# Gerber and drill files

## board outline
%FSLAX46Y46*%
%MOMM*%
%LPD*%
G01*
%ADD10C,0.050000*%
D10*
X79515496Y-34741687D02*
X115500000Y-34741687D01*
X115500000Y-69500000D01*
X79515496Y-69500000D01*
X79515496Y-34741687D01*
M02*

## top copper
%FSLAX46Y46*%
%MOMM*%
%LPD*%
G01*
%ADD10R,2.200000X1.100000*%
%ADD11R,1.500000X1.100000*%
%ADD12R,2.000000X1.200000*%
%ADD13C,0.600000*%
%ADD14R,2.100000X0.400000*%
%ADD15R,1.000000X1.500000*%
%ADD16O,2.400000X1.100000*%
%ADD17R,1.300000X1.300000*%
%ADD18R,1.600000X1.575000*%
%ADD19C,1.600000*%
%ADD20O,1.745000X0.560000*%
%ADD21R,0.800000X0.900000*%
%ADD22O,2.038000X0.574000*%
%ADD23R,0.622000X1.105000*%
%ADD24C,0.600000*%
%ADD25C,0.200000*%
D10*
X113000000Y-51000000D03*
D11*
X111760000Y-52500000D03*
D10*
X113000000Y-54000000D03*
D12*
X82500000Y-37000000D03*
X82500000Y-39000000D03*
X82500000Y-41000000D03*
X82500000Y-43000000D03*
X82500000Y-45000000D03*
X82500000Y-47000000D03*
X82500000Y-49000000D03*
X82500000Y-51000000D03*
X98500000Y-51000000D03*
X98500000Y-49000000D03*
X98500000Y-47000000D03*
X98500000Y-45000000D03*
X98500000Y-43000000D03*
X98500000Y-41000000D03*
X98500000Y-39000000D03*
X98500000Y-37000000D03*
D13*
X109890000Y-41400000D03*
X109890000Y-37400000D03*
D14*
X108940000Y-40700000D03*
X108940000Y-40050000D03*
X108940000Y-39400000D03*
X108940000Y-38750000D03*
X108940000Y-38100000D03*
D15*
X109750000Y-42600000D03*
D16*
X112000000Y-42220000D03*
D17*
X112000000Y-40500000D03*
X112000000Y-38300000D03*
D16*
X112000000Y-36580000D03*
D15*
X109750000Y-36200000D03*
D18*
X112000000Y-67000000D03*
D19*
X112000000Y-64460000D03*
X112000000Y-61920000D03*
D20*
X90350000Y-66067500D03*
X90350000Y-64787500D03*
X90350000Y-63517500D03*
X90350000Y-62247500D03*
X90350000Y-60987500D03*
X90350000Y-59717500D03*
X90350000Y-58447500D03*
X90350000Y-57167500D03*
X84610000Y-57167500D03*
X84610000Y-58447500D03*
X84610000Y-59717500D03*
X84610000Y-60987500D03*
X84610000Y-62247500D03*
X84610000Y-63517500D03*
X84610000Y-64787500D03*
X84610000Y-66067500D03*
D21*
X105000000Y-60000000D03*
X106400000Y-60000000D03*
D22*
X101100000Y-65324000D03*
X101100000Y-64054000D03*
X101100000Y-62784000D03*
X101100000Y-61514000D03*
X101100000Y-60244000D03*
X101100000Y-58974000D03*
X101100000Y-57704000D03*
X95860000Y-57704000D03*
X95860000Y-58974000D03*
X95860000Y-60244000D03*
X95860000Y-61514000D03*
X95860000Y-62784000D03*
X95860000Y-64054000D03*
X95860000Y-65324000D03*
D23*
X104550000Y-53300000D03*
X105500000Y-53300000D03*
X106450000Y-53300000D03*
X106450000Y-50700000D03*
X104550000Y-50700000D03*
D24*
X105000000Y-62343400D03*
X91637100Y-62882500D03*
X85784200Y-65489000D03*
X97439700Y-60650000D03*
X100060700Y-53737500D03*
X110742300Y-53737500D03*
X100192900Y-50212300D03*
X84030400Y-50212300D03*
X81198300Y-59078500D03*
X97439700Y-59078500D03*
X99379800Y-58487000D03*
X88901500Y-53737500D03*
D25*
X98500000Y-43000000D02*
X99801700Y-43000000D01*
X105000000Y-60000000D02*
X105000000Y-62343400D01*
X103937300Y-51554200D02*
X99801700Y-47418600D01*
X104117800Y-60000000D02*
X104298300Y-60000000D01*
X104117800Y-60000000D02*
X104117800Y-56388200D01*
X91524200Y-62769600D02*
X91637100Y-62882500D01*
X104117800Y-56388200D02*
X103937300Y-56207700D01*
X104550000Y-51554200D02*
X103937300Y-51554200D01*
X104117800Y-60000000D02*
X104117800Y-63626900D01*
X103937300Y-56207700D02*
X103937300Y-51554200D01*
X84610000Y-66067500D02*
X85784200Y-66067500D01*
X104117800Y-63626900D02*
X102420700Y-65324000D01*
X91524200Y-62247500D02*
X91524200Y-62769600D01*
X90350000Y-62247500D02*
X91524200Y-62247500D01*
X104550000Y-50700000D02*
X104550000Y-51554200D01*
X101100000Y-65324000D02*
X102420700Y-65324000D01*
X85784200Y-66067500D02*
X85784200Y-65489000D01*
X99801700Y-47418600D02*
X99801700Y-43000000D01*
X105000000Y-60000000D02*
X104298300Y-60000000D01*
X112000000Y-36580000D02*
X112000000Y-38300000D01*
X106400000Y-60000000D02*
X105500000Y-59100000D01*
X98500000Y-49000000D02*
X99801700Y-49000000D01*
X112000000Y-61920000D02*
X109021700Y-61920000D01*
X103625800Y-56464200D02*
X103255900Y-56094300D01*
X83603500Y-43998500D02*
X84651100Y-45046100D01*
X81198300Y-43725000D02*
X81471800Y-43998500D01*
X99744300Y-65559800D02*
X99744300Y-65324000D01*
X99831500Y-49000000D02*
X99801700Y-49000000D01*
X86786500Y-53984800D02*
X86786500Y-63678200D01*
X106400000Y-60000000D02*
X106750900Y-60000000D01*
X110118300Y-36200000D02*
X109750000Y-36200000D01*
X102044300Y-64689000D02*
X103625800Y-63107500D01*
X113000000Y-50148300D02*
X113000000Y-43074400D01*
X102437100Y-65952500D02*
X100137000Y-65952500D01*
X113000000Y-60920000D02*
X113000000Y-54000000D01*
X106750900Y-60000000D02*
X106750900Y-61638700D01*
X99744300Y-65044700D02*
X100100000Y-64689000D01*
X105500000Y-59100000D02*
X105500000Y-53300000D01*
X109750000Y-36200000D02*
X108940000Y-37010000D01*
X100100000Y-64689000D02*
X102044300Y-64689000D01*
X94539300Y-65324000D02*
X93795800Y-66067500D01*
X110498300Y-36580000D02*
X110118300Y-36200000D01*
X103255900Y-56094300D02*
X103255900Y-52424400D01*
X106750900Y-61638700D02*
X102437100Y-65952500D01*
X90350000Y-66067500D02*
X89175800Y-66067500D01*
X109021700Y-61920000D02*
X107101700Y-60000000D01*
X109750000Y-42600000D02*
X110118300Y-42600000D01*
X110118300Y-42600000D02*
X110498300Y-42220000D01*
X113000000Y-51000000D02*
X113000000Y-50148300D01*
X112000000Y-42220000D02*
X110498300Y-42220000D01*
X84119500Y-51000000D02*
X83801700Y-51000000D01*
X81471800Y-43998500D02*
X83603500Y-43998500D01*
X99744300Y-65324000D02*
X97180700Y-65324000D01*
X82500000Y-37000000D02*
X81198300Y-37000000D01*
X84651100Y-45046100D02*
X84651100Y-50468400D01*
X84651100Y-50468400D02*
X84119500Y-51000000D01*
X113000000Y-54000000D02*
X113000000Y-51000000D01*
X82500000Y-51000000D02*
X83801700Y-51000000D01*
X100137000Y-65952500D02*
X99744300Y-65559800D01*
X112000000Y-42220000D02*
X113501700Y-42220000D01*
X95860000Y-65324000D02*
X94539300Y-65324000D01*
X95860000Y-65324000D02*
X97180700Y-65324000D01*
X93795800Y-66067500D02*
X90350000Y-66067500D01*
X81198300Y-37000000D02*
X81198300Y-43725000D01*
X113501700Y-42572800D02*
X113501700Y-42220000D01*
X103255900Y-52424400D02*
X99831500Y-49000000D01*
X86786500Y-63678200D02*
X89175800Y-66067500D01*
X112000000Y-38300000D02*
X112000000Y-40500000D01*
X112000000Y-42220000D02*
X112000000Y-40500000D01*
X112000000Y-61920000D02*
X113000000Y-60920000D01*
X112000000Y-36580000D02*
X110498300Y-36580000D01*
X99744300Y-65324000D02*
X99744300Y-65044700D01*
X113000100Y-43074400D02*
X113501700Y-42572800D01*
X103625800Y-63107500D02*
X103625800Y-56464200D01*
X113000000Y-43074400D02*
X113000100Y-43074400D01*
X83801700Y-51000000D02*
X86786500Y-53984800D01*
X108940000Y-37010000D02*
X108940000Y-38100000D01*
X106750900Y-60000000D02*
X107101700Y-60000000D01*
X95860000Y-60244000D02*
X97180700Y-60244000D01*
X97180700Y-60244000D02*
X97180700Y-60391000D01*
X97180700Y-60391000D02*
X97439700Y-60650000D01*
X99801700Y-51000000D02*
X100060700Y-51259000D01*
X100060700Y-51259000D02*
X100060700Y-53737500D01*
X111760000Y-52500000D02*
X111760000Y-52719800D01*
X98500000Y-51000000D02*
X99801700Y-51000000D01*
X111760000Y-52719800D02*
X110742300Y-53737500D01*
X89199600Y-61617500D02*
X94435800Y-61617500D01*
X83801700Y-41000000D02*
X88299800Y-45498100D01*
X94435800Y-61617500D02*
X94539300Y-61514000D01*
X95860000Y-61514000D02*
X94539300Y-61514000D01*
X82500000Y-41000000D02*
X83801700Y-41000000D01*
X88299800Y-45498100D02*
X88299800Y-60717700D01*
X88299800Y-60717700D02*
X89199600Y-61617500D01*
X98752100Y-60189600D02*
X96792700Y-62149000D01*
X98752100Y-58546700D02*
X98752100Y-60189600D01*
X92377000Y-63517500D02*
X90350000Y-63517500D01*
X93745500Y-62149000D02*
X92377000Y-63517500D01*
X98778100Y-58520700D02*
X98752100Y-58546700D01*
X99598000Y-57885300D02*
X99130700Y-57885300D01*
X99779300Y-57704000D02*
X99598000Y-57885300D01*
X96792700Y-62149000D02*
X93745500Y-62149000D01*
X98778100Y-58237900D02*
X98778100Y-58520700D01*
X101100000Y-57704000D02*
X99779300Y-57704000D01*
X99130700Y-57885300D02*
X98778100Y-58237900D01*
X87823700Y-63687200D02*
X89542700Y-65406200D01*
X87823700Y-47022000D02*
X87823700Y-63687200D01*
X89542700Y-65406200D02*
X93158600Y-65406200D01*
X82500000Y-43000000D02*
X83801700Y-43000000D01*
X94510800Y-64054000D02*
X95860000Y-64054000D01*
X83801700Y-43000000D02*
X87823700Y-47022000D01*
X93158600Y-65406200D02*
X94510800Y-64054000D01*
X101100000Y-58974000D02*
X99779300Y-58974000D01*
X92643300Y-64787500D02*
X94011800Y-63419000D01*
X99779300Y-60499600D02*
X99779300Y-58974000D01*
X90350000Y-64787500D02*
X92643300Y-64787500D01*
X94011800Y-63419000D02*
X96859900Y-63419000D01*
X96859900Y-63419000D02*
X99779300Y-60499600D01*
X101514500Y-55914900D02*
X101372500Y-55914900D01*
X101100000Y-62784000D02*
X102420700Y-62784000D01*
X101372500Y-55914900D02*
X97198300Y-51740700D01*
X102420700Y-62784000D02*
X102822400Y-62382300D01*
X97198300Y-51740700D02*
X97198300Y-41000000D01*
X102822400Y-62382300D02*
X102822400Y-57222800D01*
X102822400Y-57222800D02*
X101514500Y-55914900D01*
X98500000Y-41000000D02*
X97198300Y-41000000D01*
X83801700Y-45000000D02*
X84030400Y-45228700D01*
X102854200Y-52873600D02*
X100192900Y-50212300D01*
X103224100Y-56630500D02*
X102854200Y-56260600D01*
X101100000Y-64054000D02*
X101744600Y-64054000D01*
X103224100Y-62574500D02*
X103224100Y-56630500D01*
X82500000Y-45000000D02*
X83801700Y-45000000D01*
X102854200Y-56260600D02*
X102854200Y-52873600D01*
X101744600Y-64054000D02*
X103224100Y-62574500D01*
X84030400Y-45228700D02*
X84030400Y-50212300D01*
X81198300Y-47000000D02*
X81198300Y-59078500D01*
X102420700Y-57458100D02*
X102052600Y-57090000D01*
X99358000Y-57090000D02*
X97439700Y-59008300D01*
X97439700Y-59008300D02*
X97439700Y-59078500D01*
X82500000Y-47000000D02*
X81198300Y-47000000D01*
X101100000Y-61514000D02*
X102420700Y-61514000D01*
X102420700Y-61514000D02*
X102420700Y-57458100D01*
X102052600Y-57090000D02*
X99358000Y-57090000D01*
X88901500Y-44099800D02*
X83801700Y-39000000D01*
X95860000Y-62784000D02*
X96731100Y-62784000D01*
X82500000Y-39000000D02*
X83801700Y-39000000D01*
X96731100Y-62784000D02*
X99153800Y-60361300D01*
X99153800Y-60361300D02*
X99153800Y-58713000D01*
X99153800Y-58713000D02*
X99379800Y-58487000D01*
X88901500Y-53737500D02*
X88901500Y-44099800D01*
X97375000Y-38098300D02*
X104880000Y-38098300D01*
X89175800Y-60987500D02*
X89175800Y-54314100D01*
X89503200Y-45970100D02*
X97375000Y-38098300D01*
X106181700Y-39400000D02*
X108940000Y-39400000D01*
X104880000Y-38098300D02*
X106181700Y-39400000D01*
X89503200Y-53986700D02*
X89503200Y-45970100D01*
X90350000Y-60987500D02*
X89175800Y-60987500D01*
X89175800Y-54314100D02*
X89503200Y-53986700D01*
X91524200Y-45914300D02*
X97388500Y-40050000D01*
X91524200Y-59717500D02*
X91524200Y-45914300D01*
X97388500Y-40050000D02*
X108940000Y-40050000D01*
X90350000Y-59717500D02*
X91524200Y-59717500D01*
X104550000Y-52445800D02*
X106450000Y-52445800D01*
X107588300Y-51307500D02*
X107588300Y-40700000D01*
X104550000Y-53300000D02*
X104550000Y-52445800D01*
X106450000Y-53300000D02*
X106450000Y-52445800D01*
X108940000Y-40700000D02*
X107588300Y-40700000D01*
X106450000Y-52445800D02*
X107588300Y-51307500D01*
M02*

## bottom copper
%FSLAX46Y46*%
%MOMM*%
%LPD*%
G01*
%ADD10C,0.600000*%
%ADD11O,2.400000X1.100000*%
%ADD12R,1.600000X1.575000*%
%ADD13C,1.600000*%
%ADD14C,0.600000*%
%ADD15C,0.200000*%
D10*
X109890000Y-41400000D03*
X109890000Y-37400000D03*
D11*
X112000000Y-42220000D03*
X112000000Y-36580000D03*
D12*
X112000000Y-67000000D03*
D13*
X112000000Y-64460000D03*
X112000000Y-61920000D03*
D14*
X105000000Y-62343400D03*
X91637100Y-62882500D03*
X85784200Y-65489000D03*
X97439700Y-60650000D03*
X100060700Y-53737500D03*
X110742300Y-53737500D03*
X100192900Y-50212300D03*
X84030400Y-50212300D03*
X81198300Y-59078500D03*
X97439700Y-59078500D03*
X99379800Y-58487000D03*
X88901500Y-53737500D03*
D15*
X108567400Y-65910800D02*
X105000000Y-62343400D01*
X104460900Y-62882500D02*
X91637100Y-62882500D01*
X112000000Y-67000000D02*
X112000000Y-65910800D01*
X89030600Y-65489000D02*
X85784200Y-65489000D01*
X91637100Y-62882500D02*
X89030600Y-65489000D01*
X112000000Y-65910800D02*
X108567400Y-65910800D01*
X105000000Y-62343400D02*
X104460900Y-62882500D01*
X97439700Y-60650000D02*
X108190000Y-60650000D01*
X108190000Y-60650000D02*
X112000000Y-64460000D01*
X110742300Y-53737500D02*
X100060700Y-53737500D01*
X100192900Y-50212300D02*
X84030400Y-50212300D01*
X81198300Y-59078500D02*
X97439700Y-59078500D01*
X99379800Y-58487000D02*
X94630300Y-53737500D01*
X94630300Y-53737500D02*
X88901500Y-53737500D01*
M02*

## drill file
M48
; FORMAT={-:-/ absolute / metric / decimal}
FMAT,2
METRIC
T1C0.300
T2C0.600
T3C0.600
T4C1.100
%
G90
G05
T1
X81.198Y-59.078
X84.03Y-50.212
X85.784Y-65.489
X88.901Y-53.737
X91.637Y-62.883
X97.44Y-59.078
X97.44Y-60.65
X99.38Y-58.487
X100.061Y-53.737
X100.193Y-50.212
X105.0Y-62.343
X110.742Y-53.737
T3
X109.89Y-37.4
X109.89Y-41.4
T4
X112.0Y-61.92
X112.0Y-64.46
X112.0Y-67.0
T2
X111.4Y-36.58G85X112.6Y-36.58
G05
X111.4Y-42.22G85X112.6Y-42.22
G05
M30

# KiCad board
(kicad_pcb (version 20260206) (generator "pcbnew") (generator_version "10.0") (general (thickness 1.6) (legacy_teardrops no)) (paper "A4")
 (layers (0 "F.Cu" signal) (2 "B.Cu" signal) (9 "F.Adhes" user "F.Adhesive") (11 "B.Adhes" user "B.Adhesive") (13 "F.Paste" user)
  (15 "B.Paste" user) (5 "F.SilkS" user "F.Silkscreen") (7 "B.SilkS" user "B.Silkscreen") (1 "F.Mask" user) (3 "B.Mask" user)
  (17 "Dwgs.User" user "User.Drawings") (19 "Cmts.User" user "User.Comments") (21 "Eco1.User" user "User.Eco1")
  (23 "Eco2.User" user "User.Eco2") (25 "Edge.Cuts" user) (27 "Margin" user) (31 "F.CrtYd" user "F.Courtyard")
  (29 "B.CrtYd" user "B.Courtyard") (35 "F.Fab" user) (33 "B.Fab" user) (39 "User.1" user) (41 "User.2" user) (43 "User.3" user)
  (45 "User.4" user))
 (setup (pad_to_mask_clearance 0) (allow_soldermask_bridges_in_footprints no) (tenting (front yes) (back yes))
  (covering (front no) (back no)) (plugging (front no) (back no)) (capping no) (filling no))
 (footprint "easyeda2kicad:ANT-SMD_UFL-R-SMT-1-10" (layer "F.Cu") (at 112.38 52.5)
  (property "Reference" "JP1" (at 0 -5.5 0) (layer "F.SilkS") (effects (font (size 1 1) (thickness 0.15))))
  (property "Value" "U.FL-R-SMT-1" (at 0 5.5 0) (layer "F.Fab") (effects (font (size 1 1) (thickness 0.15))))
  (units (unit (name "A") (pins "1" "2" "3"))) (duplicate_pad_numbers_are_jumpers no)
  (pad "1" smd rect (at 0.62 -1.5 270) (size 1.1 2.2) (layers "F.Cu" "F.Mask" "F.Paste") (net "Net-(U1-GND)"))
  (pad "2" smd rect (at -0.62 0) (size 1.5 1.1) (layers "F.Cu" "F.Mask" "F.Paste") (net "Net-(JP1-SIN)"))
  (pad "3" smd rect (at 0.62 1.5 270) (size 1.1 2.2) (layers "F.Cu" "F.Mask" "F.Paste") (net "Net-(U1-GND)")))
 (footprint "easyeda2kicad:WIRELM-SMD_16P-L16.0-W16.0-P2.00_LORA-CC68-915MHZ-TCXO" (layer "F.Cu") (at 90.5 44)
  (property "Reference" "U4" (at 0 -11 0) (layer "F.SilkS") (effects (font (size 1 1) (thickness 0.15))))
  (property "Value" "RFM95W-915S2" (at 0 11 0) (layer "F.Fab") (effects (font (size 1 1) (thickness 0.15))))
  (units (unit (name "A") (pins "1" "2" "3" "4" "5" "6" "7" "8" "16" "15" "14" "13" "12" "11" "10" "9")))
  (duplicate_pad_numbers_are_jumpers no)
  (pad "1" smd rect (at -8 -7 90) (size 1.2 2) (layers "F.Cu" "F.Mask" "F.Paste") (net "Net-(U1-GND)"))
  (pad "2" smd rect (at -8 -5 90) (size 1.2 2) (layers "F.Cu" "F.Mask" "F.Paste") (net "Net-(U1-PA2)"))
  (pad "3" smd rect (at -8 -3 90) (size 1.2 2) (layers "F.Cu" "F.Mask" "F.Paste") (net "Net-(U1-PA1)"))
  (pad "4" smd rect (at -8 -1 90) (size 1.2 2) (layers "F.Cu" "F.Mask" "F.Paste") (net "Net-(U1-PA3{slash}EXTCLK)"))
  (pad "5" smd rect (at -8 1 90) (size 1.2 2) (layers "F.Cu" "F.Mask" "F.Paste") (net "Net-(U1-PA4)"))
  (pad "6" smd rect (at -8 3 90) (size 1.2 2) (layers "F.Cu" "F.Mask" "F.Paste") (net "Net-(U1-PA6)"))
  (pad "7" smd rect (at -8 5 90) (size 1.2 2) (layers "F.Cu" "F.Mask" "F.Paste") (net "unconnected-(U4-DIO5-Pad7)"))
  (pad "8" smd rect (at -8 7 90) (size 1.2 2) (layers "F.Cu" "F.Mask" "F.Paste") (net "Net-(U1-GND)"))
  (pad "9" smd rect (at 8 7 90) (size 1.2 2) (layers "F.Cu" "F.Mask" "F.Paste") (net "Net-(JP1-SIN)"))
  (pad "10" smd rect (at 8 5 90) (size 1.2 2) (layers "F.Cu" "F.Mask" "F.Paste") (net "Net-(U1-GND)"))
  (pad "11" smd rect (at 8 3 90) (size 1.2 2) (layers "F.Cu" "F.Mask" "F.Paste") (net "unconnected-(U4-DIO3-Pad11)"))
  (pad "12" smd rect (at 8 1 90) (size 1.2 2) (layers "F.Cu" "F.Mask" "F.Paste") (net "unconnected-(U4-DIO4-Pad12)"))
  (pad "13" smd rect (at 8 -1 90) (size 1.2 2) (layers "F.Cu" "F.Mask" "F.Paste") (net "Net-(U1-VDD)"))
  (pad "14" smd rect (at 8 -3 90) (size 1.2 2) (layers "F.Cu" "F.Mask" "F.Paste") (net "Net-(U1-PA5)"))
  (pad "15" smd rect (at 8 -5 90) (size 1.2 2) (layers "F.Cu" "F.Mask" "F.Paste") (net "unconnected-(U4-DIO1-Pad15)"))
  (pad "16" smd rect (at 8 -7 90) (size 1.2 2) (layers "F.Cu" "F.Mask" "F.Paste") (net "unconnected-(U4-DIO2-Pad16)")))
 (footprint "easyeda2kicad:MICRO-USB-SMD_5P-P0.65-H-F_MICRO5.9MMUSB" (layer "F.Cu") (at 110.47 39.4 90)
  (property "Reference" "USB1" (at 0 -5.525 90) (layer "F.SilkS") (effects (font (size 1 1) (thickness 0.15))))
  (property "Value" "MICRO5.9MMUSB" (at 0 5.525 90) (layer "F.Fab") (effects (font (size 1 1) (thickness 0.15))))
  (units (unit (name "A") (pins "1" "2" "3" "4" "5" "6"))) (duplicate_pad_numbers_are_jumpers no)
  (pad "" thru_hole circle (at -2 -0.58 90) (size 0.6 0.6) (drill 0.6) (layers "*.Cu" "*.Mask") (remove_unused_layers no))
  (pad "" thru_hole circle (at 2 -0.58 90) (size 0.6 0.6) (drill 0.6) (layers "*.Cu" "*.Mask") (remove_unused_layers no))
  (pad "1" smd rect (at -1.3 -1.53 90) (size 0.4 2.1) (layers "F.Cu" "F.Mask" "F.Paste") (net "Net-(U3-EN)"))
  (pad "2" smd rect (at -0.65 -1.53 90) (size 0.4 2.1) (layers "F.Cu" "F.Mask" "F.Paste") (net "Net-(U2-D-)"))
  (pad "3" smd rect (at 0 -1.53 90) (size 0.4 2.1) (layers "F.Cu" "F.Mask" "F.Paste") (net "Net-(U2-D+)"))
  (pad "4" smd rect (at 0.65 -1.53 90) (size 0.4 2.1) (layers "F.Cu" "F.Mask" "F.Paste") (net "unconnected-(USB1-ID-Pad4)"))
  (pad "5" smd rect (at 1.3 -1.53 90) (size 0.4 2.1) (layers "F.Cu" "F.Mask" "F.Paste") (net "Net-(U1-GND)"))
  (pad "6" smd rect (at -3.2 -0.72 90) (size 1.5 1) (layers "F.Cu" "F.Mask" "F.Paste") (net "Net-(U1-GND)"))
  (pad "6" thru_hole oval (at -2.82 1.53 90) (size 1.1 2.4) (drill oval 0.599998 1.799996) (layers "*.Cu" "*.Mask")
   (remove_unused_layers no) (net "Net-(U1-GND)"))
  (pad "6" smd rect (at -1.1 1.53 90) (size 1.3 1.3) (layers "F.Cu" "F.Mask" "F.Paste") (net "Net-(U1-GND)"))
  (pad "6" smd rect (at 1.1 1.53 90) (size 1.3 1.3) (layers "F.Cu" "F.Mask" "F.Paste") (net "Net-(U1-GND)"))
  (pad "6" thru_hole oval (at 2.82 1.53 90) (size 1.1 2.4) (drill oval 0.599998 1.799996) (layers "*.Cu" "*.Mask") (remove_unused_layers no)
   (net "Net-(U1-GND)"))
  (pad "6" smd rect (at 3.2 -0.72 90) (size 1.5 1) (layers "F.Cu" "F.Mask" "F.Paste") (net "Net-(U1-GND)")))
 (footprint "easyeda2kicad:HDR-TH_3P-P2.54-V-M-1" (layer "F.Cu") (at 112 64.46 90)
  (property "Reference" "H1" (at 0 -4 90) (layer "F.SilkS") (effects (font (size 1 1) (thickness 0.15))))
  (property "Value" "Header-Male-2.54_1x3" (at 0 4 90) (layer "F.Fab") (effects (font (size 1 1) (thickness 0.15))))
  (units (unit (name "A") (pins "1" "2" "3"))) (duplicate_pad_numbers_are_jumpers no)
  (pad "1" thru_hole rect (at -2.54 0 90) (size 1.575 1.6) (drill 1.100024) (layers "*.Cu" "*.Mask") (remove_unused_layers no)
   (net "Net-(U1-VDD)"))
  (pad "2" thru_hole circle (at 0 0 90) (size 1.6 1.6) (drill 1.100024) (layers "*.Cu" "*.Mask") (remove_unused_layers no)
   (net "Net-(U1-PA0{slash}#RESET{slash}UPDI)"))
  (pad "3" thru_hole circle (at 2.54 0 90) (size 1.6 1.6) (drill 1.100024) (layers "*.Cu" "*.Mask") (remove_unused_layers no)
   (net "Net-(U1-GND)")))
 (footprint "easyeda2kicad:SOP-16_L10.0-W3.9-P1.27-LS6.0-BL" (layer "F.Cu") (at 87.48 61.6175 90)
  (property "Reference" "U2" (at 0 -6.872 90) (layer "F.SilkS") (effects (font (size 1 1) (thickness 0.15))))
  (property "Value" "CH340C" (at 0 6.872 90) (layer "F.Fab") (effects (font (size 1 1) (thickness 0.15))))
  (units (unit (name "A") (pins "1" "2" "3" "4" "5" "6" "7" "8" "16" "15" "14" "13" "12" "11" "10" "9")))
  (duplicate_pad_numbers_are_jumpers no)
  (pad "1" smd oval (at -4.45 2.87 90) (size 0.56 1.745) (layers "F.Cu" "F.Mask" "F.Paste") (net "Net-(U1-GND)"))
  (pad "2" smd oval (at -3.17 2.87 90) (size 0.56 1.745) (layers "F.Cu" "F.Mask" "F.Paste") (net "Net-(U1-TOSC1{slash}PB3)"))
  (pad "3" smd oval (at -1.9 2.87 90) (size 0.56 1.745) (layers "F.Cu" "F.Mask" "F.Paste") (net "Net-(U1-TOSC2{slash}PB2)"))
  (pad "4" smd oval (at -0.63 2.87 90) (size 0.56 1.745) (layers "F.Cu" "F.Mask" "F.Paste") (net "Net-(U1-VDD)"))
  (pad "5" smd oval (at 0.63 2.87 90) (size 0.56 1.745) (layers "F.Cu" "F.Mask" "F.Paste") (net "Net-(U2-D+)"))
  (pad "6" smd oval (at 1.9 2.87 90) (size 0.56 1.745) (layers "F.Cu" "F.Mask" "F.Paste") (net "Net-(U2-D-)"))
  (pad "7" smd oval (at 3.17 2.87 90) (size 0.56 1.745) (layers "F.Cu" "F.Mask" "F.Paste") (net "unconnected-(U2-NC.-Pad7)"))
  (pad "8" smd oval (at 4.45 2.87 90) (size 0.56 1.745) (layers "F.Cu" "F.Mask" "F.Paste") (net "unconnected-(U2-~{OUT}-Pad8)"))
  (pad "9" smd oval (at 4.45 -2.87 90) (size 0.56 1.745) (layers "F.Cu" "F.Mask" "F.Paste") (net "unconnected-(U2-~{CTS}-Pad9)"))
  (pad "10" smd oval (at 3.17 -2.87 90) (size 0.56 1.745) (layers "F.Cu" "F.Mask" "F.Paste") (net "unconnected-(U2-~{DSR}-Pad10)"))
  (pad "11" smd oval (at 1.9 -2.87 90) (size 0.56 1.745) (layers "F.Cu" "F.Mask" "F.Paste") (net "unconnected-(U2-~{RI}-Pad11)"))
  (pad "12" smd oval (at 0.63 -2.87 90) (size 0.56 1.745) (layers "F.Cu" "F.Mask" "F.Paste") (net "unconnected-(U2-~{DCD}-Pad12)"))
  (pad "13" smd oval (at -0.63 -2.87 90) (size 0.56 1.745) (layers "F.Cu" "F.Mask" "F.Paste") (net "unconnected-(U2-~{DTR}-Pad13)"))
  (pad "14" smd oval (at -1.9 -2.87 90) (size 0.56 1.745) (layers "F.Cu" "F.Mask" "F.Paste") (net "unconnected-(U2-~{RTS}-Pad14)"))
  (pad "15" smd oval (at -3.17 -2.87 90) (size 0.56 1.745) (layers "F.Cu" "F.Mask" "F.Paste") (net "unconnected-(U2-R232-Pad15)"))
  (pad "16" smd oval (at -4.45 -2.87 90) (size 0.56 1.745) (layers "F.Cu" "F.Mask" "F.Paste") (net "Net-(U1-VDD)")))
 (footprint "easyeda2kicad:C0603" (layer "F.Cu") (at 105.7 60)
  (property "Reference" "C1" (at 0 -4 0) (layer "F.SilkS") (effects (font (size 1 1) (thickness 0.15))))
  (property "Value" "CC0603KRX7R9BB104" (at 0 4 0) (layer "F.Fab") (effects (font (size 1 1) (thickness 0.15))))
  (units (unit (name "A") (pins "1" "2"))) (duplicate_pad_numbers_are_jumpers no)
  (pad "1" smd rect (at -0.7 0) (size 0.8 0.9) (layers "F.Cu" "F.Mask" "F.Paste") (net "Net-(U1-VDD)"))
  (pad "2" smd rect (at 0.7 0) (size 0.8 0.9) (layers "F.Cu" "F.Mask" "F.Paste") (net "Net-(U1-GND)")))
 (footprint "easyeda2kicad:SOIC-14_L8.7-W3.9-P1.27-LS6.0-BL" (layer "F.Cu") (at 98.48 61.514 90)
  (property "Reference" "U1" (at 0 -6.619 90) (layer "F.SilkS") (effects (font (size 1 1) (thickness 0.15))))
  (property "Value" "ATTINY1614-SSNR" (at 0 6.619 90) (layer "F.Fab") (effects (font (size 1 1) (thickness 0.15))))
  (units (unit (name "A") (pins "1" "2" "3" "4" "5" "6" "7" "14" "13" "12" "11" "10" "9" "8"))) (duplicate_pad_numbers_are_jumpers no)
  (pad "1" smd oval (at -3.81 2.62 90) (size 0.574 2.038) (layers "F.Cu" "F.Mask" "F.Paste") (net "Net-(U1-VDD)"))
  (pad "2" smd oval (at -2.54 2.62 90) (size 0.574 2.038) (layers "F.Cu" "F.Mask" "F.Paste") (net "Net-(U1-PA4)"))
  (pad "3" smd oval (at -1.27 2.62 90) (size 0.574 2.038) (layers "F.Cu" "F.Mask" "F.Paste") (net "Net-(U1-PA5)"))
  (pad "4" smd oval (at 0 2.62 90) (size 0.574 2.038) (layers "F.Cu" "F.Mask" "F.Paste") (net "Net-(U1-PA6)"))
  (pad "5" smd oval (at 1.27 2.62 90) (size 0.574 2.038) (layers "F.Cu" "F.Mask" "F.Paste") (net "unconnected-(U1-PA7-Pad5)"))
  (pad "6" smd oval (at 2.54 2.62 90) (size 0.574 2.038) (layers "F.Cu" "F.Mask" "F.Paste") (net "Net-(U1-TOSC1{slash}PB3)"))
  (pad "7" smd oval (at 3.81 2.62 90) (size 0.574 2.038) (layers "F.Cu" "F.Mask" "F.Paste") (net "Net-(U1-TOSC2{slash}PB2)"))
  (pad "8" smd oval (at 3.81 -2.62 90) (size 0.574 2.038) (layers "F.Cu" "F.Mask" "F.Paste") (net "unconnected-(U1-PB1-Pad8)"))
  (pad "9" smd oval (at 2.54 -2.62 90) (size 0.574 2.038) (layers "F.Cu" "F.Mask" "F.Paste") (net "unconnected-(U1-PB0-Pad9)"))
  (pad "10" smd oval (at 1.27 -2.62 90) (size 0.574 2.038) (layers "F.Cu" "F.Mask" "F.Paste") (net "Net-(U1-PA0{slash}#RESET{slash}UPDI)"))
  (pad "11" smd oval (at 0 -2.62 90) (size 0.574 2.038) (layers "F.Cu" "F.Mask" "F.Paste") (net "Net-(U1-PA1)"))
  (pad "12" smd oval (at -1.27 -2.62 90) (size 0.574 2.038) (layers "F.Cu" "F.Mask" "F.Paste") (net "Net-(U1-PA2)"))
  (pad "13" smd oval (at -2.54 -2.62 90) (size 0.574 2.038) (layers "F.Cu" "F.Mask" "F.Paste") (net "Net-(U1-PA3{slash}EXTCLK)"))
  (pad "14" smd oval (at -3.81 -2.62 90) (size 0.574 2.038) (layers "F.Cu" "F.Mask" "F.Paste") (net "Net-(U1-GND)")))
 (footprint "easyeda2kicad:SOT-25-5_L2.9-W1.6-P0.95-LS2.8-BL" (layer "F.Cu") (at 105.5 52)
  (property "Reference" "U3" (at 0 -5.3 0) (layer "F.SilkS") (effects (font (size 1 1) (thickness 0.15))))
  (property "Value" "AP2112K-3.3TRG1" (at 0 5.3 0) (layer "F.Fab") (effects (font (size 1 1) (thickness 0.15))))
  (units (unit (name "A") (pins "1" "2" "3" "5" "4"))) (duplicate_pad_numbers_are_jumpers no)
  (pad "1" smd rect (at -0.95 1.3) (size 0.622 1.105) (layers "F.Cu" "F.Mask" "F.Paste") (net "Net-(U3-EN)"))
  (pad "2" smd rect (at 0 1.3) (size 0.622 1.105) (layers "F.Cu" "F.Mask" "F.Paste") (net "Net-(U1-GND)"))
  (pad "3" smd rect (at 0.95 1.3) (size 0.622 1.105) (layers "F.Cu" "F.Mask" "F.Paste") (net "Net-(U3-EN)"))
  (pad "4" smd rect (at 0.95 -1.3) (size 0.622 1.105) (layers "F.Cu" "F.Mask" "F.Paste") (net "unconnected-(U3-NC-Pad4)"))
  (pad "5" smd rect (at -0.95 -1.3) (size 0.622 1.105) (layers "F.Cu" "F.Mask" "F.Paste") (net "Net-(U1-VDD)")))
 (gr_rect (start 79.515496 34.741687) (end 115.5 69.5) (stroke (width 0.05) (type default)) (fill no) (layer "Edge.Cuts"))
 (segment (start 98.5 43) (end 99.8017 43) (width 0.2) (layer "F.Cu") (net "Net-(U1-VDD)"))
 (segment (start 105 60) (end 105 62.3434) (width 0.2) (layer "F.Cu") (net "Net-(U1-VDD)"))
 (segment (start 103.9373 51.5542) (end 99.8017 47.4186) (width 0.2) (layer "F.Cu") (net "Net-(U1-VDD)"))
 (segment (start 104.1178 60) (end 104.2983 60) (width 0.2) (layer "F.Cu") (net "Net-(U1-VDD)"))
 (segment (start 104.1178 60) (end 104.1178 56.3882) (width 0.2) (layer "F.Cu") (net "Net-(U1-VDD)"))
 (segment (start 91.5242 62.7696) (end 91.6371 62.8825) (width 0.2) (layer "F.Cu") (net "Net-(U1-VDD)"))
 (segment (start 104.1178 56.3882) (end 103.9373 56.2077) (width 0.2) (layer "F.Cu") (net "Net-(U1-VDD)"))
 (segment (start 104.55 51.5542) (end 103.9373 51.5542) (width 0.2) (layer "F.Cu") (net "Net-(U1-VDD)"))
 (segment (start 104.1178 60) (end 104.1178 63.6269) (width 0.2) (layer "F.Cu") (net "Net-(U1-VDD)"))
 (segment (start 103.9373 56.2077) (end 103.9373 51.5542) (width 0.2) (layer "F.Cu") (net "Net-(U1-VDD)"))
 (segment (start 84.61 66.0675) (end 85.7842 66.0675) (width 0.2) (layer "F.Cu") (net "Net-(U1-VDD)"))
 (segment (start 104.1178 63.6269) (end 102.4207 65.324) (width 0.2) (layer "F.Cu") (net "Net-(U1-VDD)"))
 (segment (start 91.5242 62.2475) (end 91.5242 62.7696) (width 0.2) (layer "F.Cu") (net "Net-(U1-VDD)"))
 (segment (start 90.35 62.2475) (end 91.5242 62.2475) (width 0.2) (layer "F.Cu") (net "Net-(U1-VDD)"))
 (segment (start 104.55 50.7) (end 104.55 51.5542) (width 0.2) (layer "F.Cu") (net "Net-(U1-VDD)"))
 (segment (start 101.1 65.324) (end 102.4207 65.324) (width 0.2) (layer "F.Cu") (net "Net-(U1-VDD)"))
 (segment (start 85.7842 66.0675) (end 85.7842 65.489) (width 0.2) (layer "F.Cu") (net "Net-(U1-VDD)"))
 (segment (start 99.8017 47.4186) (end 99.8017 43) (width 0.2) (layer "F.Cu") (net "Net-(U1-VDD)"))
 (segment (start 105 60) (end 104.2983 60) (width 0.2) (layer "F.Cu") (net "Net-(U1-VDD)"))
 (via (at 105 62.3434) (size 0.6) (drill 0.3) (layers "F.Cu" "B.Cu") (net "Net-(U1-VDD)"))
 (via (at 91.6371 62.8825) (size 0.6) (drill 0.3) (layers "F.Cu" "B.Cu") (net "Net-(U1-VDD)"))
 (via (at 85.7842 65.489) (size 0.6) (drill 0.3) (layers "F.Cu" "B.Cu") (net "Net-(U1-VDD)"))
 (segment (start 108.5674 65.9108) (end 105 62.3434) (width 0.2) (layer "B.Cu") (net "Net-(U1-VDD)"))
 (segment (start 104.4609 62.8825) (end 91.6371 62.8825) (width 0.2) (layer "B.Cu") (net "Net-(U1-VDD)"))
 (segment (start 112 67) (end 112 65.9108) (width 0.2) (layer "B.Cu") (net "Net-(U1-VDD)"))
 (segment (start 89.0306 65.489) (end 85.7842 65.489) (width 0.2) (layer "B.Cu") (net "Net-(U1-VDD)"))
 (segment (start 91.6371 62.8825) (end 89.0306 65.489) (width 0.2) (layer "B.Cu") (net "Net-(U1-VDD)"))
 (segment (start 112 65.9108) (end 108.5674 65.9108) (width 0.2) (layer "B.Cu") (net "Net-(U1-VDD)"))
 (segment (start 105 62.3434) (end 104.4609 62.8825) (width 0.2) (layer "B.Cu") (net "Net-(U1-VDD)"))
 (segment (start 112 36.58) (end 112 38.3) (width 0.2) (layer "F.Cu") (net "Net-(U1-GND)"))
 (segment (start 106.4 60) (end 105.5 59.1) (width 0.2) (layer "F.Cu") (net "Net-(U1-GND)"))
 (segment (start 98.5 49) (end 99.8017 49) (width 0.2) (layer "F.Cu") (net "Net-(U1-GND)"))
 (segment (start 112 61.92) (end 109.0217 61.92) (width 0.2) (layer "F.Cu") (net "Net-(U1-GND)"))
 (segment (start 103.6258 56.4642) (end 103.2559 56.0943) (width 0.2) (layer "F.Cu") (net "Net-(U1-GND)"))
 (segment (start 83.6035 43.9985) (end 84.6511 45.0461) (width 0.2) (layer "F.Cu") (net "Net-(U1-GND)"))
 (segment (start 81.1983 43.725) (end 81.4718 43.9985) (width 0.2) (layer "F.Cu") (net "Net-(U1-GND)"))
 (segment (start 99.7443 65.5598) (end 99.7443 65.324) (width 0.2) (layer "F.Cu") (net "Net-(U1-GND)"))
 (segment (start 99.8315 49) (end 99.8017 49) (width 0.2) (layer "F.Cu") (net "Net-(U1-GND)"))
 (segment (start 86.7865 53.9848) (end 86.7865 63.6782) (width 0.2) (layer "F.Cu") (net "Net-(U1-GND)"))
 (segment (start 106.4 60) (end 106.7509 60) (width 0.2) (layer "F.Cu") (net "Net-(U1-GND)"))
 (segment (start 110.1183 36.2) (end 109.75 36.2) (width 0.2) (layer "F.Cu") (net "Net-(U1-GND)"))
 (segment (start 102.0443 64.689) (end 103.6258 63.1075) (width 0.2) (layer "F.Cu") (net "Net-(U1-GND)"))
 (segment (start 113 50.1483) (end 113 43.0744) (width 0.2) (layer "F.Cu") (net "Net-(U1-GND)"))
 (segment (start 102.4371 65.9525) (end 100.137 65.9525) (width 0.2) (layer "F.Cu") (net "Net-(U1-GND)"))
 (segment (start 113 60.92) (end 113 54) (width 0.2) (layer "F.Cu") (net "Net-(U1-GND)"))
 (segment (start 106.7509 60) (end 106.7509 61.6387) (width 0.2) (layer "F.Cu") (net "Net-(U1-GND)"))
 (segment (start 99.7443 65.0447) (end 100.1 64.689) (width 0.2) (layer "F.Cu") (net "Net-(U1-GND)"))
 (segment (start 105.5 59.1) (end 105.5 53.3) (width 0.2) (layer "F.Cu") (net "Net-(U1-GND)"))
 (segment (start 109.75 36.2) (end 108.94 37.01) (width 0.2) (layer "F.Cu") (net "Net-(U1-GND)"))
 (segment (start 100.1 64.689) (end 102.0443 64.689) (width 0.2) (layer "F.Cu") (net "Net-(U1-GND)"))
 (segment (start 94.5393 65.324) (end 93.7958 66.0675) (width 0.2) (layer "F.Cu") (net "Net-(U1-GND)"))
 (segment (start 110.4983 36.58) (end 110.1183 36.2) (width 0.2) (layer "F.Cu") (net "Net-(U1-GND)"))
 (segment (start 103.2559 56.0943) (end 103.2559 52.4244) (width 0.2) (layer "F.Cu") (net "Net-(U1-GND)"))
 (segment (start 106.7509 61.6387) (end 102.4371 65.9525) (width 0.2) (layer "F.Cu") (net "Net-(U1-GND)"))
 (segment (start 90.35 66.0675) (end 89.1758 66.0675) (width 0.2) (layer "F.Cu") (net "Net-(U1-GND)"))
 (segment (start 109.0217 61.92) (end 107.1017 60) (width 0.2) (layer "F.Cu") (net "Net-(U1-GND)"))
 (segment (start 109.75 42.6) (end 110.1183 42.6) (width 0.2) (layer "F.Cu") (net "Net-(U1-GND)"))
 (segment (start 110.1183 42.6) (end 110.4983 42.22) (width 0.2) (layer "F.Cu") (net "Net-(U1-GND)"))
 (segment (start 113 51) (end 113 50.1483) (width 0.2) (layer "F.Cu") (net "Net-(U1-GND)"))
 (segment (start 112 42.22) (end 110.4983 42.22) (width 0.2) (layer "F.Cu") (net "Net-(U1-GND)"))
 (segment (start 84.1195 51) (end 83.8017 51) (width 0.2) (layer "F.Cu") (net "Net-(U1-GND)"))
 (segment (start 81.4718 43.9985) (end 83.6035 43.9985) (width 0.2) (layer "F.Cu") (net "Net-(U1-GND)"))
 (segment (start 99.7443 65.324) (end 97.1807 65.324) (width 0.2) (layer "F.Cu") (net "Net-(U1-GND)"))
 (segment (start 82.5 37) (end 81.1983 37) (width 0.2) (layer "F.Cu") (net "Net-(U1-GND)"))
 (segment (start 84.6511 45.0461) (end 84.6511 50.4684) (width 0.2) (layer "F.Cu") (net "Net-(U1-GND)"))
 (segment (start 84.6511 50.4684) (end 84.1195 51) (width 0.2) (layer "F.Cu") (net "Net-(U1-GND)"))
 (segment (start 113 54) (end 113 51) (width 0.2) (layer "F.Cu") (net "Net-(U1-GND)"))
 (segment (start 82.5 51) (end 83.8017 51) (width 0.2) (layer "F.Cu") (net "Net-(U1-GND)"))
 (segment (start 100.137 65.9525) (end 99.7443 65.5598) (width 0.2) (layer "F.Cu") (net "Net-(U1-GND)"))
 (segment (start 112 42.22) (end 113.5017 42.22) (width 0.2) (layer "F.Cu") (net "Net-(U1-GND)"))
 (segment (start 95.86 65.324) (end 94.5393 65.324) (width 0.2) (layer "F.Cu") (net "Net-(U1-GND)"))
 (segment (start 95.86 65.324) (end 97.1807 65.324) (width 0.2) (layer "F.Cu") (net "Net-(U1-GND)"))
 (segment (start 93.7958 66.0675) (end 90.35 66.0675) (width 0.2) (layer "F.Cu") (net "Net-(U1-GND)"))
 (segment (start 81.1983 37) (end 81.1983 43.725) (width 0.2) (layer "F.Cu") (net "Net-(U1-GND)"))
 (segment (start 113.5017 42.5728) (end 113.5017 42.22) (width 0.2) (layer "F.Cu") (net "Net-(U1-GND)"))
 (segment (start 103.2559 52.4244) (end 99.8315 49) (width 0.2) (layer "F.Cu") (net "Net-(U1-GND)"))
 (segment (start 86.7865 63.6782) (end 89.1758 66.0675) (width 0.2) (layer "F.Cu") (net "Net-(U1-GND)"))
 (segment (start 112 38.3) (end 112 40.5) (width 0.2) (layer "F.Cu") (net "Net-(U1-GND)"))
 (segment (start 112 42.22) (end 112 40.5) (width 0.2) (layer "F.Cu") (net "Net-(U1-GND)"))
 (segment (start 112 61.92) (end 113 60.92) (width 0.2) (layer "F.Cu") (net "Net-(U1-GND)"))
 (segment (start 112 36.58) (end 110.4983 36.58) (width 0.2) (layer "F.Cu") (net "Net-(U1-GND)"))
 (segment (start 99.7443 65.324) (end 99.7443 65.0447) (width 0.2) (layer "F.Cu") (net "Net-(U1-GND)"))
 (segment (start 113.0001 43.0744) (end 113.5017 42.5728) (width 0.2) (layer "F.Cu") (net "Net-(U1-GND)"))
 (segment (start 103.6258 63.1075) (end 103.6258 56.4642) (width 0.2) (layer "F.Cu") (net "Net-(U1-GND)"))
 (segment (start 113 43.0744) (end 113.0001 43.0744) (width 0.2) (layer "F.Cu") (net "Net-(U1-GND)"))
 (segment (start 83.8017 51) (end 86.7865 53.9848) (width 0.2) (layer "F.Cu") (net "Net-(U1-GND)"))
 (segment (start 108.94 37.01) (end 108.94 38.1) (width 0.2) (layer "F.Cu") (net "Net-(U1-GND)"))
 (segment (start 106.7509 60) (end 107.1017 60) (width 0.2) (layer "F.Cu") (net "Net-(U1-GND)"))
 (segment (start 95.86 60.244) (end 97.1807 60.244) (width 0.2) (layer "F.Cu") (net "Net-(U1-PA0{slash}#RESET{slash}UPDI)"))
 (segment (start 97.1807 60.244) (end 97.1807 60.391) (width 0.2) (layer "F.Cu") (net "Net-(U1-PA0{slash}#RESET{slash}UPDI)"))
 (segment (start 97.1807 60.391) (end 97.4397 60.65) (width 0.2) (layer "F.Cu") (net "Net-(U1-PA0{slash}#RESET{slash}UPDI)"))
 (via (at 97.4397 60.65) (size 0.6) (drill 0.3) (layers "F.Cu" "B.Cu") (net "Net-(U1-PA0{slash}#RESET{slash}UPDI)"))
 (segment (start 97.4397 60.65) (end 108.19 60.65) (width 0.2) (layer "B.Cu") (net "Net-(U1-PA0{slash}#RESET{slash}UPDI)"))
 (segment (start 108.19 60.65) (end 112 64.46) (width 0.2) (layer "B.Cu") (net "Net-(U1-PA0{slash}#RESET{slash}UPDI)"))
 (segment (start 99.8017 51) (end 100.0607 51.259) (width 0.2) (layer "F.Cu") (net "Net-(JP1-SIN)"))
 (segment (start 100.0607 51.259) (end 100.0607 53.7375) (width 0.2) (layer "F.Cu") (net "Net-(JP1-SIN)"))
 (segment (start 111.76 52.5) (end 111.76 52.7198) (width 0.2) (layer "F.Cu") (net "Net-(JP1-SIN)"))
 (segment (start 98.5 51) (end 99.8017 51) (width 0.2) (layer "F.Cu") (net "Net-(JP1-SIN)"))
 (segment (start 111.76 52.7198) (end 110.7423 53.7375) (width 0.2) (layer "F.Cu") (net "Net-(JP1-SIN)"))
 (via (at 100.0607 53.7375) (size 0.6) (drill 0.3) (layers "F.Cu" "B.Cu") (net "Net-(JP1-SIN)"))
 (via (at 110.7423 53.7375) (size 0.6) (drill 0.3) (layers "F.Cu" "B.Cu") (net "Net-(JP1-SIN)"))
 (segment (start 110.7423 53.7375) (end 100.0607 53.7375) (width 0.2) (layer "B.Cu") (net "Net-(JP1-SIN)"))
 (segment (start 89.1996 61.6175) (end 94.4358 61.6175) (width 0.2) (layer "F.Cu") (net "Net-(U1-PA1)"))
 (segment (start 83.8017 41) (end 88.2998 45.4981) (width 0.2) (layer "F.Cu") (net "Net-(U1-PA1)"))
 (segment (start 94.4358 61.6175) (end 94.5393 61.514) (width 0.2) (layer "F.Cu") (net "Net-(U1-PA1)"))
 (segment (start 95.86 61.514) (end 94.5393 61.514) (width 0.2) (layer "F.Cu") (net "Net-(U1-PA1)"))
 (segment (start 82.5 41) (end 83.8017 41) (width 0.2) (layer "F.Cu") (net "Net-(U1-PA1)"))
 (segment (start 88.2998 45.4981) (end 88.2998 60.7177) (width 0.2) (layer "F.Cu") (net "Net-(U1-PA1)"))
 (segment (start 88.2998 60.7177) (end 89.1996 61.6175) (width 0.2) (layer "F.Cu") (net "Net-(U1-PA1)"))
 (segment (start 98.7521 60.1896) (end 96.7927 62.149) (width 0.2) (layer "F.Cu") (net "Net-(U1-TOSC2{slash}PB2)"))
 (segment (start 98.7521 58.5467) (end 98.7521 60.1896) (width 0.2) (layer "F.Cu") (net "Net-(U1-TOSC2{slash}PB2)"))
 (segment (start 92.377 63.5175) (end 90.35 63.5175) (width 0.2) (layer "F.Cu") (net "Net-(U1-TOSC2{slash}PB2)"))
 (segment (start 93.7455 62.149) (end 92.377 63.5175) (width 0.2) (layer "F.Cu") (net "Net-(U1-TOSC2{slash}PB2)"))
 (segment (start 98.7781 58.5207) (end 98.7521 58.5467) (width 0.2) (layer "F.Cu") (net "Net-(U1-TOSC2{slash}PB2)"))
 (segment (start 99.598 57.8853) (end 99.1307 57.8853) (width 0.2) (layer "F.Cu") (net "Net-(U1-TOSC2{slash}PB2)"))
 (segment (start 99.7793 57.704) (end 99.598 57.8853) (width 0.2) (layer "F.Cu") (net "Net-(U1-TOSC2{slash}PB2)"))
 (segment (start 96.7927 62.149) (end 93.7455 62.149) (width 0.2) (layer "F.Cu") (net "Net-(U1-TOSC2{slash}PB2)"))
 (segment (start 98.7781 58.2379) (end 98.7781 58.5207) (width 0.2) (layer "F.Cu") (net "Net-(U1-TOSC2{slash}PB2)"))
 (segment (start 101.1 57.704) (end 99.7793 57.704) (width 0.2) (layer "F.Cu") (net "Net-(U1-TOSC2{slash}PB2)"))
 (segment (start 99.1307 57.8853) (end 98.7781 58.2379) (width 0.2) (layer "F.Cu") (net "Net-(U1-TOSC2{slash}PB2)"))
 (segment (start 87.8237 63.6872) (end 89.5427 65.4062) (width 0.2) (layer "F.Cu") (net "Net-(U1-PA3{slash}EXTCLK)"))
 (segment (start 87.8237 47.022) (end 87.8237 63.6872) (width 0.2) (layer "F.Cu") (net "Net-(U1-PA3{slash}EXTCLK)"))
 (segment (start 89.5427 65.4062) (end 93.1586 65.4062) (width 0.2) (layer "F.Cu") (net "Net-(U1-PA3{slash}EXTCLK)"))
 (segment (start 82.5 43) (end 83.8017 43) (width 0.2) (layer "F.Cu") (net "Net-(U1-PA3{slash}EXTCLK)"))
 (segment (start 94.5108 64.054) (end 95.86 64.054) (width 0.2) (layer "F.Cu") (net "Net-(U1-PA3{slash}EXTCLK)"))
 (segment (start 83.8017 43) (end 87.8237 47.022) (width 0.2) (layer "F.Cu") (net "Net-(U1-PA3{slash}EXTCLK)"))
 (segment (start 93.1586 65.4062) (end 94.5108 64.054) (width 0.2) (layer "F.Cu") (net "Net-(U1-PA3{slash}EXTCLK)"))
 (segment (start 101.1 58.974) (end 99.7793 58.974) (width 0.2) (layer "F.Cu") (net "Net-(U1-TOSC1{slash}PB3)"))
 (segment (start 92.6433 64.7875) (end 94.0118 63.419) (width 0.2) (layer "F.Cu") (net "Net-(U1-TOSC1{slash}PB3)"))
 (segment (start 99.7793 60.4996) (end 99.7793 58.974) (width 0.2) (layer "F.Cu") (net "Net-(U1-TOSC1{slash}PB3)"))
 (segment (start 90.35 64.7875) (end 92.6433 64.7875) (width 0.2) (layer "F.Cu") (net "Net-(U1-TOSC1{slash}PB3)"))
 (segment (start 94.0118 63.419) (end 96.8599 63.419) (width 0.2) (layer "F.Cu") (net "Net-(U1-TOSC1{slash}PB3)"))
 (segment (start 96.8599 63.419) (end 99.7793 60.4996) (width 0.2) (layer "F.Cu") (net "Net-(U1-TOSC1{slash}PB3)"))
 (segment (start 101.5145 55.9149) (end 101.3725 55.9149) (width 0.2) (layer "F.Cu") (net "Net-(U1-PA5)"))
 (segment (start 101.1 62.784) (end 102.4207 62.784) (width 0.2) (layer "F.Cu") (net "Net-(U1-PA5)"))
 (segment (start 101.3725 55.9149) (end 97.1983 51.7407) (width 0.2) (layer "F.Cu") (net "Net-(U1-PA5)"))
 (segment (start 102.4207 62.784) (end 102.8224 62.3823) (width 0.2) (layer "F.Cu") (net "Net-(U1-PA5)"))
 (segment (start 97.1983 51.7407) (end 97.1983 41) (width 0.2) (layer "F.Cu") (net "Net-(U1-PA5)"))
 (segment (start 102.8224 62.3823) (end 102.8224 57.2228) (width 0.2) (layer "F.Cu") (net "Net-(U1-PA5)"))
 (segment (start 102.8224 57.2228) (end 101.5145 55.9149) (width 0.2) (layer "F.Cu") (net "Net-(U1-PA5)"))
 (segment (start 98.5 41) (end 97.1983 41) (width 0.2) (layer "F.Cu") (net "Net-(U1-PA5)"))
 (segment (start 83.8017 45) (end 84.0304 45.2287) (width 0.2) (layer "F.Cu") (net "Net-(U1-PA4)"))
 (segment (start 102.8542 52.8736) (end 100.1929 50.2123) (width 0.2) (layer "F.Cu") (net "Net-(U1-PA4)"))
 (segment (start 103.2241 56.6305) (end 102.8542 56.2606) (width 0.2) (layer "F.Cu") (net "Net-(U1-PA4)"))
 (segment (start 101.1 64.054) (end 101.7446 64.054) (width 0.2) (layer "F.Cu") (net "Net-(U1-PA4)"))
 (segment (start 103.2241 62.5745) (end 103.2241 56.6305) (width 0.2) (layer "F.Cu") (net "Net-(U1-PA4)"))
 (segment (start 82.5 45) (end 83.8017 45) (width 0.2) (layer "F.Cu") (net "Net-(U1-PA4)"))
 (segment (start 102.8542 56.2606) (end 102.8542 52.8736) (width 0.2) (layer "F.Cu") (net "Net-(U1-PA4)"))
 (segment (start 101.7446 64.054) (end 103.2241 62.5745) (width 0.2) (layer "F.Cu") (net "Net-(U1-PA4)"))
 (segment (start 84.0304 45.2287) (end 84.0304 50.2123) (width 0.2) (layer "F.Cu") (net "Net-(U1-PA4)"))
 (via (at 100.1929 50.2123) (size 0.6) (drill 0.3) (layers "F.Cu" "B.Cu") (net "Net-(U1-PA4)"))
 (via (at 84.0304 50.2123) (size 0.6) (drill 0.3) (layers "F.Cu" "B.Cu") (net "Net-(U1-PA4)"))
 (segment (start 100.1929 50.2123) (end 84.0304 50.2123) (width 0.2) (layer "B.Cu") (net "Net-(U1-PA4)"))
 (segment (start 81.1983 47) (end 81.1983 59.0785) (width 0.2) (layer "F.Cu") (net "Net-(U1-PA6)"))
 (segment (start 102.4207 57.4581) (end 102.0526 57.09) (width 0.2) (layer "F.Cu") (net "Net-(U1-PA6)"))
 (segment (start 99.358 57.09) (end 97.4397 59.0083) (width 0.2) (layer "F.Cu") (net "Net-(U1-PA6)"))
 (segment (start 97.4397 59.0083) (end 97.4397 59.0785) (width 0.2) (layer "F.Cu") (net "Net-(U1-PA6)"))
 (segment (start 82.5 47) (end 81.1983 47) (width 0.2) (layer "F.Cu") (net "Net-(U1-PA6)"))
 (segment (start 101.1 61.514) (end 102.4207 61.514) (width 0.2) (layer "F.Cu") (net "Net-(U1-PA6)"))
 (segment (start 102.4207 61.514) (end 102.4207 57.4581) (width 0.2) (layer "F.Cu") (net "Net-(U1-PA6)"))
 (segment (start 102.0526 57.09) (end 99.358 57.09) (width 0.2) (layer "F.Cu") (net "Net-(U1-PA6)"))
 (via (at 81.1983 59.0785) (size 0.6) (drill 0.3) (layers "F.Cu" "B.Cu") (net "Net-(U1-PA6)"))
 (via (at 97.4397 59.0785) (size 0.6) (drill 0.3) (layers "F.Cu" "B.Cu") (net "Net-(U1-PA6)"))
 (segment (start 81.1983 59.0785) (end 97.4397 59.0785) (width 0.2) (layer "B.Cu") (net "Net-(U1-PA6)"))
 (segment (start 88.9015 44.0998) (end 83.8017 39) (width 0.2) (layer "F.Cu") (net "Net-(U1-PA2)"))
 (segment (start 95.86 62.784) (end 96.7311 62.784) (width 0.2) (layer "F.Cu") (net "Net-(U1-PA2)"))
 (segment (start 82.5 39) (end 83.8017 39) (width 0.2) (layer "F.Cu") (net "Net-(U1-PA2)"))
 (segment (start 96.7311 62.784) (end 99.1538 60.3613) (width 0.2) (layer "F.Cu") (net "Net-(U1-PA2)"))
 (segment (start 99.1538 60.3613) (end 99.1538 58.713) (width 0.2) (layer "F.Cu") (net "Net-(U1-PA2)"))
 (segment (start 99.1538 58.713) (end 99.3798 58.487) (width 0.2) (layer "F.Cu") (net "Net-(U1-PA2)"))
 (segment (start 88.9015 53.7375) (end 88.9015 44.0998) (width 0.2) (layer "F.Cu") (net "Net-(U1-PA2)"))
 (via (at 99.3798 58.487) (size 0.6) (drill 0.3) (layers "F.Cu" "B.Cu") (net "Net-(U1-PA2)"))
 (via (at 88.9015 53.7375) (size 0.6) (drill 0.3) (layers "F.Cu" "B.Cu") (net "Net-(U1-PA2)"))
 (segment (start 99.3798 58.487) (end 94.6303 53.7375) (width 0.2) (layer "B.Cu") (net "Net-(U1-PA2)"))
 (segment (start 94.6303 53.7375) (end 88.9015 53.7375) (width 0.2) (layer "B.Cu") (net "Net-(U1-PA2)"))
 (segment (start 97.375 38.0983) (end 104.88 38.0983) (width 0.2) (layer "F.Cu") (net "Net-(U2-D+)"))
 (segment (start 89.1758 60.9875) (end 89.1758 54.3141) (width 0.2) (layer "F.Cu") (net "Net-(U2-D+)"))
 (segment (start 89.5032 45.9701) (end 97.375 38.0983) (width 0.2) (layer "F.Cu") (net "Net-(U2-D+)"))
 (segment (start 106.1817 39.4) (end 108.94 39.4) (width 0.2) (layer "F.Cu") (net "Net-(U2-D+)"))
 (segment (start 104.88 38.0983) (end 106.1817 39.4) (width 0.2) (layer "F.Cu") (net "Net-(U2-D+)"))
 (segment (start 89.5032 53.9867) (end 89.5032 45.9701) (width 0.2) (layer "F.Cu") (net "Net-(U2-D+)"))
 (segment (start 90.35 60.9875) (end 89.1758 60.9875) (width 0.2) (layer "F.Cu") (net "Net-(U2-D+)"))
 (segment (start 89.1758 54.3141) (end 89.5032 53.9867) (width 0.2) (layer "F.Cu") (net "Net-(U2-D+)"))
 (segment (start 91.5242 45.9143) (end 97.3885 40.05) (width 0.2) (layer "F.Cu") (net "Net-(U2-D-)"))
 (segment (start 91.5242 59.7175) (end 91.5242 45.9143) (width 0.2) (layer "F.Cu") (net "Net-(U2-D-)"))
 (segment (start 97.3885 40.05) (end 108.94 40.05) (width 0.2) (layer "F.Cu") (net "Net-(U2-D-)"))
 (segment (start 90.35 59.7175) (end 91.5242 59.7175) (width 0.2) (layer "F.Cu") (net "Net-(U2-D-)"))
 (segment (start 104.55 52.4458) (end 106.45 52.4458) (width 0.2) (layer "F.Cu") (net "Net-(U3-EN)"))
 (segment (start 107.5883 51.3075) (end 107.5883 40.7) (width 0.2) (layer "F.Cu") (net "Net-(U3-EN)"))
 (segment (start 104.55 53.3) (end 104.55 52.4458) (width 0.2) (layer "F.Cu") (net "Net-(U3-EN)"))
 (segment (start 106.45 53.3) (end 106.45 52.4458) (width 0.2) (layer "F.Cu") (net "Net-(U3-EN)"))
 (segment (start 108.94 40.7) (end 107.5883 40.7) (width 0.2) (layer "F.Cu") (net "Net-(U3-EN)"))
 (segment (start 106.45 52.4458) (end 107.5883 51.3075) (width 0.2) (layer "F.Cu") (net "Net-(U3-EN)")))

